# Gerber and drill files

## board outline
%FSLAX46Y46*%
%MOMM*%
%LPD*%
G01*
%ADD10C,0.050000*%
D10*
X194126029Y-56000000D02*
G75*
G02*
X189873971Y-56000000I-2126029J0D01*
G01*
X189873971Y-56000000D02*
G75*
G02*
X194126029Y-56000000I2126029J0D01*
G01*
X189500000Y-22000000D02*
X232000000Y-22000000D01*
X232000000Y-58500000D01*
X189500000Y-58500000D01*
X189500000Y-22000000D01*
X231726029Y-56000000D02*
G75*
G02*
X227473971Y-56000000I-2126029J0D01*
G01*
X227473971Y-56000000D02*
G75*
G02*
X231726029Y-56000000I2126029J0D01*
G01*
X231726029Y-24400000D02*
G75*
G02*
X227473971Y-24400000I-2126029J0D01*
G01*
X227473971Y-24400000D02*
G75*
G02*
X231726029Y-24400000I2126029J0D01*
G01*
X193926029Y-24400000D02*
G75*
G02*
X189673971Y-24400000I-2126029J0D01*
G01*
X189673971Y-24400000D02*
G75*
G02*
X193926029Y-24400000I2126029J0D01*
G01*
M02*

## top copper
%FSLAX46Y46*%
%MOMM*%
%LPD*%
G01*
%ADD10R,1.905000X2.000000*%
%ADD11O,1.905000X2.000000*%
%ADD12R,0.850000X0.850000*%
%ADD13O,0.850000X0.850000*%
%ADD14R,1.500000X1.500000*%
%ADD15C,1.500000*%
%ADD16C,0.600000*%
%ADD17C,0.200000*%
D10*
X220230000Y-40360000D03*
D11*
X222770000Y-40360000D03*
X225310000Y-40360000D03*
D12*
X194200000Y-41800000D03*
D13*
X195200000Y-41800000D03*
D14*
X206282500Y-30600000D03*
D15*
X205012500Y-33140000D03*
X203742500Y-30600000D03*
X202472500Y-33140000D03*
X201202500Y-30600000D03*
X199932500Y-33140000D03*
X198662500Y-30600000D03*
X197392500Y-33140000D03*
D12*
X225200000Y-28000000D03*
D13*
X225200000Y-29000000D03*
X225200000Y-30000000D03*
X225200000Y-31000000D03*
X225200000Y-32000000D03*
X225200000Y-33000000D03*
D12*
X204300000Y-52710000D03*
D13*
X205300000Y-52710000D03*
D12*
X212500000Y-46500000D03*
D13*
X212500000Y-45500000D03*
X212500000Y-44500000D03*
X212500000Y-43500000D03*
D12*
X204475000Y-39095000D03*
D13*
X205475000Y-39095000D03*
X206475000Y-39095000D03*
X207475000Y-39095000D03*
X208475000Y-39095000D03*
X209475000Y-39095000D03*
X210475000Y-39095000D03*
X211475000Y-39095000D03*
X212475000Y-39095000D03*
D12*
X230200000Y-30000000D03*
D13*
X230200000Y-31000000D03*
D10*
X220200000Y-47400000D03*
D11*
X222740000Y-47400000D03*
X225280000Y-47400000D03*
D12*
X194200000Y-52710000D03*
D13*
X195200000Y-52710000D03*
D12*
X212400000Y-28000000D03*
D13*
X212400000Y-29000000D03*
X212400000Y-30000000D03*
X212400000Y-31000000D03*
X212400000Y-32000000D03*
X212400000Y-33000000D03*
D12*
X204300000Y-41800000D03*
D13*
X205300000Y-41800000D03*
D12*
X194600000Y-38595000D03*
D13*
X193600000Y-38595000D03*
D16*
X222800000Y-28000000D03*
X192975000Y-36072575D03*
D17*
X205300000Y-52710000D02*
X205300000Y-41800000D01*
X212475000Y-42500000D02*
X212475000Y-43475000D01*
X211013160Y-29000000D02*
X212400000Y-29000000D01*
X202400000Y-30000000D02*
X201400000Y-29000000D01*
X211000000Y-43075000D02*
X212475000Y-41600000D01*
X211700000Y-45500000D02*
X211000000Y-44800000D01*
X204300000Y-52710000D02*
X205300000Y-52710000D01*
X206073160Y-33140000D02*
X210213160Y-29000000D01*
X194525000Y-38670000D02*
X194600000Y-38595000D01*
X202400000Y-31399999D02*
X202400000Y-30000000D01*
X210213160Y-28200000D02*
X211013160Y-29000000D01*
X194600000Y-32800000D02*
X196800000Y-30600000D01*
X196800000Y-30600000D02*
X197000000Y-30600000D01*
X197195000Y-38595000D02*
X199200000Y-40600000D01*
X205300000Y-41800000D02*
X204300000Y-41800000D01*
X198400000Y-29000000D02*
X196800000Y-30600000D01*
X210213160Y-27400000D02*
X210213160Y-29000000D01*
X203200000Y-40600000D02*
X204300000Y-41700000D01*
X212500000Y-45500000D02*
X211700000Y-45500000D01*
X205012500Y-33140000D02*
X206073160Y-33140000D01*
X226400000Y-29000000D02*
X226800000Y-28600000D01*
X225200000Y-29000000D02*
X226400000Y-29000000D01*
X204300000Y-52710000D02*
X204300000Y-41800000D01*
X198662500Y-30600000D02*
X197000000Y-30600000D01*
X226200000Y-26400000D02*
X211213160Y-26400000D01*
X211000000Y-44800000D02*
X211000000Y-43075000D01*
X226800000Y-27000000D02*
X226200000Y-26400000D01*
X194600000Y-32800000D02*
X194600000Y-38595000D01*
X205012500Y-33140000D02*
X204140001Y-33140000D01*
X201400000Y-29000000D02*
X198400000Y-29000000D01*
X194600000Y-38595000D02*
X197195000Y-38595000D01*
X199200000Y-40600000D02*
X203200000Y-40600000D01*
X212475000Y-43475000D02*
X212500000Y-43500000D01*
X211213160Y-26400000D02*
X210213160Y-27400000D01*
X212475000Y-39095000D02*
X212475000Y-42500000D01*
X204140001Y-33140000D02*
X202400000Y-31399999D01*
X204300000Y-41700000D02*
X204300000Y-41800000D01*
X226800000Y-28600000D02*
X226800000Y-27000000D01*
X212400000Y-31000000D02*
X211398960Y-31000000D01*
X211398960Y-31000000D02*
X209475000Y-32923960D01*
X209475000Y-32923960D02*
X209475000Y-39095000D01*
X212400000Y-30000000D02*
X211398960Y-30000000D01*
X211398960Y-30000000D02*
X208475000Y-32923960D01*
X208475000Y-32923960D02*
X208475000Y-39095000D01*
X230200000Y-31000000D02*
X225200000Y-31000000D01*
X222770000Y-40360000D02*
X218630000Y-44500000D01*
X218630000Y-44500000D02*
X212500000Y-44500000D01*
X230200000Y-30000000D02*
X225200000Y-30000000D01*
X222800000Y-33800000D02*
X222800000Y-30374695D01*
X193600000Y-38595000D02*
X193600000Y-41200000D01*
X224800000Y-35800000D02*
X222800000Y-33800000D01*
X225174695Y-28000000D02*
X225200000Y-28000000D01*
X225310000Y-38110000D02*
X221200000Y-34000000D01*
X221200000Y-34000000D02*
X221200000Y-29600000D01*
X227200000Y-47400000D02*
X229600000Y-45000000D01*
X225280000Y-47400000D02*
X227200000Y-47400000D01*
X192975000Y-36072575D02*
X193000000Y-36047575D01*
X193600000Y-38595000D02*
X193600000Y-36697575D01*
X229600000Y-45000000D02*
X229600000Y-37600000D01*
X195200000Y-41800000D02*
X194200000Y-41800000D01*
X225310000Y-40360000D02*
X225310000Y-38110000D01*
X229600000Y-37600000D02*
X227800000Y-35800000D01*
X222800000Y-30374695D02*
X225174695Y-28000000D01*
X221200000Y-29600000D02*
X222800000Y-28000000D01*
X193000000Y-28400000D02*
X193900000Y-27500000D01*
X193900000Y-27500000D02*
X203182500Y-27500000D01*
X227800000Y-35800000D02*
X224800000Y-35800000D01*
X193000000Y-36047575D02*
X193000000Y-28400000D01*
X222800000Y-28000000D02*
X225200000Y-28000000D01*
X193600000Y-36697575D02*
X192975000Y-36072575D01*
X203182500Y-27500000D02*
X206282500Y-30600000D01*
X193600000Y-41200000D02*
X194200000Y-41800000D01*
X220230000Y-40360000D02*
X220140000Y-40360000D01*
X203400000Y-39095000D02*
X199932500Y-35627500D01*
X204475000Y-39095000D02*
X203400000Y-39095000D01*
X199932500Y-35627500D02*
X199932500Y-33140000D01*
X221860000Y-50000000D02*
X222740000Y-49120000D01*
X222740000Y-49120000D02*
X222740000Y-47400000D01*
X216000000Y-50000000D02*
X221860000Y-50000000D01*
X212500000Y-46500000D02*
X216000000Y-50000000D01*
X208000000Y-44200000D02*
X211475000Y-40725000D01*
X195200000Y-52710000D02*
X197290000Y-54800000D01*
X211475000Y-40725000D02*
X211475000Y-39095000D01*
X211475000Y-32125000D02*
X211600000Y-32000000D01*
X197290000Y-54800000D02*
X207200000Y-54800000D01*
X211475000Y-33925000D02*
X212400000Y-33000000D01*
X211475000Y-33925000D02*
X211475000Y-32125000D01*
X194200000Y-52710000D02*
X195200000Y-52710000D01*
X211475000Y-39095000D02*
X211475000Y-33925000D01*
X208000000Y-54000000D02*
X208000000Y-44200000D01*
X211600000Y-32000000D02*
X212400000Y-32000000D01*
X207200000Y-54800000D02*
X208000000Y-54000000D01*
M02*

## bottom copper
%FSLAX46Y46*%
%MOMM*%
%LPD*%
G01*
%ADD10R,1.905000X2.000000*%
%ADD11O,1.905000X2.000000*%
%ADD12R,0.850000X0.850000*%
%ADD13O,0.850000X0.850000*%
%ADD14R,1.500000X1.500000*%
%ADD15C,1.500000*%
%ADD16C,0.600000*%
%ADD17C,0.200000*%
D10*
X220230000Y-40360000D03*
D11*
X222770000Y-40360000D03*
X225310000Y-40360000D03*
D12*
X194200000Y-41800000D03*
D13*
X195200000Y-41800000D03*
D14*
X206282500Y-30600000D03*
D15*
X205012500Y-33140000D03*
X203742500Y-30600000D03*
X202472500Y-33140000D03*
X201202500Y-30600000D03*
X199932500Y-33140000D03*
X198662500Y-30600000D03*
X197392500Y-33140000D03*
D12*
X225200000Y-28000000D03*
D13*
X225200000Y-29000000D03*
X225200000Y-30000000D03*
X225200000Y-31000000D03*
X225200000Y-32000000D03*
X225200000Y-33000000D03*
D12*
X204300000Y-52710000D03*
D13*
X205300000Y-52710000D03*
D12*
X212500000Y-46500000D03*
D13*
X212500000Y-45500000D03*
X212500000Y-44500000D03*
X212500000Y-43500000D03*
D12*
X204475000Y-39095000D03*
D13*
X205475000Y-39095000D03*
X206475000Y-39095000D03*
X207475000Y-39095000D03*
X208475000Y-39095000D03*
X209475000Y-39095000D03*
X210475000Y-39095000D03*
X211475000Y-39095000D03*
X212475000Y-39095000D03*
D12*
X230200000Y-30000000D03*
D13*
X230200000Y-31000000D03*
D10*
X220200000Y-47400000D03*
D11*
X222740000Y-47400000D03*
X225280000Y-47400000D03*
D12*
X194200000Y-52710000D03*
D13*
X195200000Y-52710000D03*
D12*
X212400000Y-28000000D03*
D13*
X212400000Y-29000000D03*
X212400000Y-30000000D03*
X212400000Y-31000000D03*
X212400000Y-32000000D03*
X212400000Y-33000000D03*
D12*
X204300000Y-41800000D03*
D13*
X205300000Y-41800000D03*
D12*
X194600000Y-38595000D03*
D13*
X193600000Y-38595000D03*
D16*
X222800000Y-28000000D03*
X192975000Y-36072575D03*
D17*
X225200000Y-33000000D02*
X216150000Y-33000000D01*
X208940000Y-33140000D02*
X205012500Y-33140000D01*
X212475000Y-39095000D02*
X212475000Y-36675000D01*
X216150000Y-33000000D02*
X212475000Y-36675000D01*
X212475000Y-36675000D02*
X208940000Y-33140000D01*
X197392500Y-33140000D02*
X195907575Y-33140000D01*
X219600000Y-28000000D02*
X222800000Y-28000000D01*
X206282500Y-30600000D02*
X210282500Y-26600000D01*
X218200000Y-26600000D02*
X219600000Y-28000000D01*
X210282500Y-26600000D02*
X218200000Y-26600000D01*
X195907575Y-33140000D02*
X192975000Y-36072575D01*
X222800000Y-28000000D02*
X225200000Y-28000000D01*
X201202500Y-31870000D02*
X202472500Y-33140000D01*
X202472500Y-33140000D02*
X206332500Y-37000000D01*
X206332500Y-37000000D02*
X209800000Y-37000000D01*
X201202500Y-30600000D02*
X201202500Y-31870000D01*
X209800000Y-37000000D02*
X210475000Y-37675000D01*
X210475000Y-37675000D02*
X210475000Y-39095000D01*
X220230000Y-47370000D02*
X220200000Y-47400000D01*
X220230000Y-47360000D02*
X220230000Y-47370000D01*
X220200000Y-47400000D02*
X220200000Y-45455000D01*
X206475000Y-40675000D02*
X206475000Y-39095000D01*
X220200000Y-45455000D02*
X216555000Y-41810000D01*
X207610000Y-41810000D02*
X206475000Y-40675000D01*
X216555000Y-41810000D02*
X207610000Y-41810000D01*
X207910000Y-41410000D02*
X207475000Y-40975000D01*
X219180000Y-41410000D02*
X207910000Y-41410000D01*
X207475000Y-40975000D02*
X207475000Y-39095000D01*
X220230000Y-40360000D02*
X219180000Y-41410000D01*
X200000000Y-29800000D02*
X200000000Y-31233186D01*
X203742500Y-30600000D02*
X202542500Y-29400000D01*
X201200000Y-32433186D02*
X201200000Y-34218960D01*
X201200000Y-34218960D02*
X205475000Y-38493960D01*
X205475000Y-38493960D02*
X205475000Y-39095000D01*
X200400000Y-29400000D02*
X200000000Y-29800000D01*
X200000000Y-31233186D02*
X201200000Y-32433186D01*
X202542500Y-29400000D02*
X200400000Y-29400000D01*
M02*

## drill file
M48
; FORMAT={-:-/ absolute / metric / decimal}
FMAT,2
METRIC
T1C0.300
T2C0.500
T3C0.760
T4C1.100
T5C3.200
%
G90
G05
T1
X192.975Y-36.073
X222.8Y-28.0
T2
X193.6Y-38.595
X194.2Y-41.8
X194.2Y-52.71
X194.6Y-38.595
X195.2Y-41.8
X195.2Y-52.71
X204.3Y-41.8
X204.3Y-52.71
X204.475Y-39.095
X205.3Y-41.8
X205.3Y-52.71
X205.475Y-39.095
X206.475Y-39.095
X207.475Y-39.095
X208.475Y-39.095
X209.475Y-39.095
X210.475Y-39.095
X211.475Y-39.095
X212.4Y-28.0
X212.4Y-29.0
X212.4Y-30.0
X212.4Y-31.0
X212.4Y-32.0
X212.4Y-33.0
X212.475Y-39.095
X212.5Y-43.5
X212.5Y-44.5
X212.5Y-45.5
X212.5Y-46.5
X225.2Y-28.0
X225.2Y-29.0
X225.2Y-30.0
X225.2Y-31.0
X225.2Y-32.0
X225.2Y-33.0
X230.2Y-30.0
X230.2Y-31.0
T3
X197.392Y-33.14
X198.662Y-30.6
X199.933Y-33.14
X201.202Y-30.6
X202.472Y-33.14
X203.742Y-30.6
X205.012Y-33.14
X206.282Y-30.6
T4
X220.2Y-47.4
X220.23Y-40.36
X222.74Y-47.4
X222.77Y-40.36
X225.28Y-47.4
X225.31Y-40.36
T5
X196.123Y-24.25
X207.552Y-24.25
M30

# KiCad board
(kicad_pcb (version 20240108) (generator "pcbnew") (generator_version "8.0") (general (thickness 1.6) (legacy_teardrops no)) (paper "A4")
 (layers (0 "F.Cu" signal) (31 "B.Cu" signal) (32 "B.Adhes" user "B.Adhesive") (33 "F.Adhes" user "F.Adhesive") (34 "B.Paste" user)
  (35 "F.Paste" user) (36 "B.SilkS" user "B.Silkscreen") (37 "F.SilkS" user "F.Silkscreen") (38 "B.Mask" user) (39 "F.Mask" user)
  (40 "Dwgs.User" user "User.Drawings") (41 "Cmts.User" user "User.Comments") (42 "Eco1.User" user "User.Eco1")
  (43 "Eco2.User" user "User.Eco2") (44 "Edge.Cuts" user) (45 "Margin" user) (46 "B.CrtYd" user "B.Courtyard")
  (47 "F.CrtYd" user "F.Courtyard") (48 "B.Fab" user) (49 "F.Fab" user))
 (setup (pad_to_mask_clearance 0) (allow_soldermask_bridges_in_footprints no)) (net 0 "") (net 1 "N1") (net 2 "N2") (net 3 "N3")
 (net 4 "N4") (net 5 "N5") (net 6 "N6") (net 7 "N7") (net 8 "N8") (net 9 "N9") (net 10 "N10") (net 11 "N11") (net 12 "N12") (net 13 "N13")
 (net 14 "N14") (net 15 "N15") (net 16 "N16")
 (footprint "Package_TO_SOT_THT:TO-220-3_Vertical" (layer "F.Cu") (at 220.23 40.36)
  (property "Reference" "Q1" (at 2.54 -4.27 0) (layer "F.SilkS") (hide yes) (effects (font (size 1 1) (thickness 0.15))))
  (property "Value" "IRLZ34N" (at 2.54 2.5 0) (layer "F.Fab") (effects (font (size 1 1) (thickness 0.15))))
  (pad "1" thru_hole rect (at 0 0) (size 1.905 2) (drill 1.1) (layers "*.Cu" "*.Mask") (remove_unused_layers no) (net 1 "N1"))
  (pad "2" thru_hole oval (at 2.54 0) (size 1.905 2) (drill 1.1) (layers "*.Cu" "*.Mask") (remove_unused_layers no) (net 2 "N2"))
  (pad "3" thru_hole oval (at 5.08 0) (size 1.905 2) (drill 1.1) (layers "*.Cu" "*.Mask") (remove_unused_layers no) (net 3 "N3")))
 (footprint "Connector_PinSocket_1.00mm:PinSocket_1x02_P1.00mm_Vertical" (layer "F.Cu") (at 194.2 41.8 90)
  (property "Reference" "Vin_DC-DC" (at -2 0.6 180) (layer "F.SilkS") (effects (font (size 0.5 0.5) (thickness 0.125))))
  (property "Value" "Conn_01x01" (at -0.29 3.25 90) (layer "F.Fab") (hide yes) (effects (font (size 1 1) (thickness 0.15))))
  (pad "1" thru_hole rect (at 0 0 90) (size 0.85 0.85) (drill 0.5) (layers "*.Cu" "*.Mask") (remove_unused_layers no) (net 3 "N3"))
  (pad "2" thru_hole oval (at 0 1 90) (size 0.85 0.85) (drill 0.5) (layers "*.Cu" "*.Mask") (remove_unused_layers no) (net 3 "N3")))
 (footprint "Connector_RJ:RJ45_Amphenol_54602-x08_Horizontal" (layer "F.Cu") (at 206.2825 30.6 180)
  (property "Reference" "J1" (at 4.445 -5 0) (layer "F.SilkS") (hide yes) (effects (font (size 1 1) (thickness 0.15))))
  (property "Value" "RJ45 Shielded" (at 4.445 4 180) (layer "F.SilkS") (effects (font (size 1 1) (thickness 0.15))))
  (pad "" np_thru_hole circle (at -1.27 6.35 180) (size 3.2 3.2) (drill 3.2) (layers "*.Cu" "*.Mask"))
  (pad "" np_thru_hole circle (at 10.16 6.35 180) (size 3.2 3.2) (drill 3.2) (layers "*.Cu" "*.Mask"))
  (pad "1" thru_hole rect (at 0 0 180) (size 1.5 1.5) (drill 0.76) (layers "*.Cu" "*.Mask") (remove_unused_layers no) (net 3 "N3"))
  (pad "2" thru_hole circle (at 1.27 -2.54 180) (size 1.5 1.5) (drill 0.76) (layers "*.Cu" "*.Mask") (remove_unused_layers no) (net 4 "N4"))
  (pad "3" thru_hole circle (at 2.54 0 180) (size 1.5 1.5) (drill 0.76) (layers "*.Cu" "*.Mask") (remove_unused_layers no) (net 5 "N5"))
  (pad "4" thru_hole circle (at 3.81 -2.54 180) (size 1.5 1.5) (drill 0.76) (layers "*.Cu" "*.Mask") (remove_unused_layers no) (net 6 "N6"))
  (pad "5" thru_hole circle (at 5.08 0 180) (size 1.5 1.5) (drill 0.76) (layers "*.Cu" "*.Mask") (remove_unused_layers no) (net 6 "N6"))
  (pad "6" thru_hole circle (at 6.35 -2.54 180) (size 1.5 1.5) (drill 0.76) (layers "*.Cu" "*.Mask") (remove_unused_layers no) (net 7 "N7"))
  (pad "7" thru_hole circle (at 7.62 0 180) (size 1.5 1.5) (drill 0.76) (layers "*.Cu" "*.Mask") (remove_unused_layers no) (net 4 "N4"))
  (pad "8" thru_hole circle (at 8.89 -2.54 180) (size 1.5 1.5) (drill 0.76) (layers "*.Cu" "*.Mask") (remove_unused_layers no) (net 3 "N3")))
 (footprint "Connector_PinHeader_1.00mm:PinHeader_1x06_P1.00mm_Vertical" (layer "F.Cu") (at 225.2 28)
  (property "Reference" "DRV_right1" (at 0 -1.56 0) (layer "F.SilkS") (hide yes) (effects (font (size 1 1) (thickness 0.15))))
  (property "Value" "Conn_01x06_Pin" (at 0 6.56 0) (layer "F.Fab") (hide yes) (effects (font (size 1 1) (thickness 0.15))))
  (pad "1" thru_hole rect (at 0 0) (size 0.85 0.85) (drill 0.5) (layers "*.Cu" "*.Mask") (remove_unused_layers no) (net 3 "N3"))
  (pad "2" thru_hole oval (at 0 1) (size 0.85 0.85) (drill 0.5) (layers "*.Cu" "*.Mask") (remove_unused_layers no) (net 4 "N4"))
  (pad "3" thru_hole oval (at 0 2) (size 0.85 0.85) (drill 0.5) (layers "*.Cu" "*.Mask") (remove_unused_layers no) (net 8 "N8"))
  (pad "4" thru_hole oval (at 0 3) (size 0.85 0.85) (drill 0.5) (layers "*.Cu" "*.Mask") (remove_unused_layers no) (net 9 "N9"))
  (pad "5" thru_hole oval (at 0 4) (size 0.85 0.85) (drill 0.5) (layers "*.Cu" "*.Mask") (remove_unused_layers no) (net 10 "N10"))
  (pad "6" thru_hole oval (at 0 5) (size 0.85 0.85) (drill 0.5) (layers "*.Cu" "*.Mask") (remove_unused_layers no) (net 4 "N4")))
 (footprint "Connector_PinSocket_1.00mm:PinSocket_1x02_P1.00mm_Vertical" (layer "F.Cu") (at 204.3 52.71 90)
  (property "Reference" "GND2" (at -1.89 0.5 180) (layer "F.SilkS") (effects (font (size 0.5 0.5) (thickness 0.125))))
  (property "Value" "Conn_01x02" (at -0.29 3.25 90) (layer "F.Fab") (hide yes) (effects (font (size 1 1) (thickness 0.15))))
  (pad "1" thru_hole rect (at 0 0 90) (size 0.85 0.85) (drill 0.5) (layers "*.Cu" "*.Mask") (remove_unused_layers no) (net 4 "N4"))
  (pad "2" thru_hole oval (at 0 1 90) (size 0.85 0.85) (drill 0.5) (layers "*.Cu" "*.Mask") (remove_unused_layers no) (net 4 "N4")))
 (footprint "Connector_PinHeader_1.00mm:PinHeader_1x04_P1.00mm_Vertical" (layer "F.Cu") (at 212.5 46.5 180)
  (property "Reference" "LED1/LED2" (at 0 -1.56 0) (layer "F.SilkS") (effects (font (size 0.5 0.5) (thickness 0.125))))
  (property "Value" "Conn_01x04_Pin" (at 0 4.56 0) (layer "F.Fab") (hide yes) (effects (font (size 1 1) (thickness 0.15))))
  (pad "1" thru_hole rect (at 0 0 180) (size 0.85 0.85) (drill 0.5) (layers "*.Cu" "*.Mask") (remove_unused_layers no) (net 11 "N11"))
  (pad "2" thru_hole oval (at 0 1 180) (size 0.85 0.85) (drill 0.5) (layers "*.Cu" "*.Mask") (remove_unused_layers no) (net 4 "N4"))
  (pad "3" thru_hole oval (at 0 2 180) (size 0.85 0.85) (drill 0.5) (layers "*.Cu" "*.Mask") (remove_unused_layers no) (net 2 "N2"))
  (pad "4" thru_hole oval (at 0 3 180) (size 0.85 0.85) (drill 0.5) (layers "*.Cu" "*.Mask") (remove_unused_layers no) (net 4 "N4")))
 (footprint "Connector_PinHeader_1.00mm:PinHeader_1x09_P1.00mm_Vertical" (layer "F.Cu") (at 204.475 39.095 90)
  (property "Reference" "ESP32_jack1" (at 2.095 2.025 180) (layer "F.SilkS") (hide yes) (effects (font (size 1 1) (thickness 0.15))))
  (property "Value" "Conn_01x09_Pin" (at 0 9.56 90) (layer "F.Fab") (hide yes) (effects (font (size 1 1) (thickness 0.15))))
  (pad "1" thru_hole rect (at 0 0 90) (size 0.85 0.85) (drill 0.5) (layers "*.Cu" "*.Mask") (remove_unused_layers no) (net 7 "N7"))
  (pad "2" thru_hole oval (at 0 1 90) (size 0.85 0.85) (drill 0.5) (layers "*.Cu" "*.Mask") (remove_unused_layers no) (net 5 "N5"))
  (pad "3" thru_hole oval (at 0 2 90) (size 0.85 0.85) (drill 0.5) (layers "*.Cu" "*.Mask") (remove_unused_layers no) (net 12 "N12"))
  (pad "4" thru_hole oval (at 0 3 90) (size 0.85 0.85) (drill 0.5) (layers "*.Cu" "*.Mask") (remove_unused_layers no) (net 1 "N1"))
  (pad "5" thru_hole oval (at 0 4 90) (size 0.85 0.85) (drill 0.5) (layers "*.Cu" "*.Mask") (remove_unused_layers no) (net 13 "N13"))
  (pad "6" thru_hole oval (at 0 5 90) (size 0.85 0.85) (drill 0.5) (layers "*.Cu" "*.Mask") (remove_unused_layers no) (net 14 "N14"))
  (pad "7" thru_hole oval (at 0 6 90) (size 0.85 0.85) (drill 0.5) (layers "*.Cu" "*.Mask") (remove_unused_layers no) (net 6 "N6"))
  (pad "8" thru_hole oval (at 0 7 90) (size 0.85 0.85) (drill 0.5) (layers "*.Cu" "*.Mask") (remove_unused_layers no) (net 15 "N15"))
  (pad "9" thru_hole oval (at 0 8 90) (size 0.85 0.85) (drill 0.5) (layers "*.Cu" "*.Mask") (remove_unused_layers no) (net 4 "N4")))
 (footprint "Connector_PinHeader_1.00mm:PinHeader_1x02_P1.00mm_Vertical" (layer "F.Cu") (at 230.2 30)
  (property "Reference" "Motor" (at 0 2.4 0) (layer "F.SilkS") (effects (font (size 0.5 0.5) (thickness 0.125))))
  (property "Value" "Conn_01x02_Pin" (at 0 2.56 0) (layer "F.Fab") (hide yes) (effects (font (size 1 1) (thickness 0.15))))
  (pad "1" thru_hole rect (at 0 0) (size 0.85 0.85) (drill 0.5) (layers "*.Cu" "*.Mask") (remove_unused_layers no) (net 8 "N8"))
  (pad "2" thru_hole oval (at 0 1) (size 0.85 0.85) (drill 0.5) (layers "*.Cu" "*.Mask") (remove_unused_layers no) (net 9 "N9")))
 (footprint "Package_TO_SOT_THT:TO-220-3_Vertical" (layer "F.Cu") (at 220.2 47.4)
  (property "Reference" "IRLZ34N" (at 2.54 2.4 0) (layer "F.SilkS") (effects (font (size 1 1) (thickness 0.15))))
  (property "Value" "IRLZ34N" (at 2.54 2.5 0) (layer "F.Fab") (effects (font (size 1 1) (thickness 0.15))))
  (pad "1" thru_hole rect (at 0 0) (size 1.905 2) (drill 1.1) (layers "*.Cu" "*.Mask") (remove_unused_layers no) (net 12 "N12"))
  (pad "2" thru_hole oval (at 2.54 0) (size 1.905 2) (drill 1.1) (layers "*.Cu" "*.Mask") (remove_unused_layers no) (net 11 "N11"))
  (pad "3" thru_hole oval (at 5.08 0) (size 1.905 2) (drill 1.1) (layers "*.Cu" "*.Mask") (remove_unused_layers no) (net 3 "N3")))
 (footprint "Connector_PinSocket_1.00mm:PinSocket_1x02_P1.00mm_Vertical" (layer "F.Cu") (at 194.2 52.71 90)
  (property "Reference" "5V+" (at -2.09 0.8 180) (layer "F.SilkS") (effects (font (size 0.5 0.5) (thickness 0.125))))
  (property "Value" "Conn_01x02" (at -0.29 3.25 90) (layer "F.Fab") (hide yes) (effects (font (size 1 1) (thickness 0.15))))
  (pad "1" thru_hole rect (at 0 0 90) (size 0.85 0.85) (drill 0.5) (layers "*.Cu" "*.Mask") (remove_unused_layers no) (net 15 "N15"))
  (pad "2" thru_hole oval (at 0 1 90) (size 0.85 0.85) (drill 0.5) (layers "*.Cu" "*.Mask") (remove_unused_layers no) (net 15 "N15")))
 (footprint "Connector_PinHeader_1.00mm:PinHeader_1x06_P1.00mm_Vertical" (layer "F.Cu") (at 212.4 28)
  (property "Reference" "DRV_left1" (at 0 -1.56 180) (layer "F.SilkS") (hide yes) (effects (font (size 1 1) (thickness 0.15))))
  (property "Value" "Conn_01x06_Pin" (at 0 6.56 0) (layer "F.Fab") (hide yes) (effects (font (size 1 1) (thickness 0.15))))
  (pad "1" thru_hole rect (at 0 0) (size 0.85 0.85) (drill 0.5) (layers "*.Cu" "*.Mask") (remove_unused_layers no) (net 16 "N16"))
  (pad "2" thru_hole oval (at 0 1) (size 0.85 0.85) (drill 0.5) (layers "*.Cu" "*.Mask") (remove_unused_layers no) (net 4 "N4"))
  (pad "3" thru_hole oval (at 0 2) (size 0.85 0.85) (drill 0.5) (layers "*.Cu" "*.Mask") (remove_unused_layers no) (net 13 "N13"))
  (pad "4" thru_hole oval (at 0 3) (size 0.85 0.85) (drill 0.5) (layers "*.Cu" "*.Mask") (remove_unused_layers no) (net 14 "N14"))
  (pad "5" thru_hole oval (at 0 4) (size 0.85 0.85) (drill 0.5) (layers "*.Cu" "*.Mask") (remove_unused_layers no) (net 15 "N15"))
  (pad "6" thru_hole oval (at 0 5) (size 0.85 0.85) (drill 0.5) (layers "*.Cu" "*.Mask") (remove_unused_layers no) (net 15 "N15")))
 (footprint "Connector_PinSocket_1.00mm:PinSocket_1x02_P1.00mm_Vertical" (layer "F.Cu") (at 204.3 41.8 90)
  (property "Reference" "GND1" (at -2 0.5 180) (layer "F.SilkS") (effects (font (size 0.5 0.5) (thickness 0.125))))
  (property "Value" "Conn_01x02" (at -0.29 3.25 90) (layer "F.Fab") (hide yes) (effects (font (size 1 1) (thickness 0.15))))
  (pad "1" thru_hole rect (at 0 0 90) (size 0.85 0.85) (drill 0.5) (layers "*.Cu" "*.Mask") (remove_unused_layers no) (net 4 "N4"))
  (pad "2" thru_hole oval (at 0 1 90) (size 0.85 0.85) (drill 0.5) (layers "*.Cu" "*.Mask") (remove_unused_layers no) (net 4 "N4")))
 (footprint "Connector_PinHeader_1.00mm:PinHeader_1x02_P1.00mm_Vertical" (layer "F.Cu") (at 194.6 38.595 -90)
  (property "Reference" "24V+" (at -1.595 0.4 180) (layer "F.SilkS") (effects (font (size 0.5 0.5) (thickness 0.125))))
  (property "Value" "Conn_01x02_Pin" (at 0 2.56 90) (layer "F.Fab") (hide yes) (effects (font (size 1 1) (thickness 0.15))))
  (pad "1" thru_hole rect (at 0 0 270) (size 0.85 0.85) (drill 0.5) (layers "*.Cu" "*.Mask") (remove_unused_layers no) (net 4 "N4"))
  (pad "2" thru_hole oval (at 0 1 270) (size 0.85 0.85) (drill 0.5) (layers "*.Cu" "*.Mask") (remove_unused_layers no) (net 3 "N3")))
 (gr_circle (center 192 56) (end 190.6 54.4) (stroke (width 0.05) (type default)) (fill none) (layer "Edge.Cuts"))
 (gr_rect (start 189.5 22) (end 232 58.5) (stroke (width 0.05) (type default)) (fill none) (layer "Edge.Cuts"))
 (gr_circle (center 229.6 56) (end 228.2 54.4) (stroke (width 0.05) (type default)) (fill none) (layer "Edge.Cuts"))
 (gr_circle (center 229.6 24.4) (end 228.2 22.8) (stroke (width 0.05) (type default)) (fill none) (layer "Edge.Cuts"))
 (gr_circle (center 191.8 24.4) (end 190.4 22.8) (stroke (width 0.05) (type default)) (fill none) (layer "Edge.Cuts"))
 (segment (start 205.3 52.71) (end 205.3 41.8) (width 0.2) (layer "F.Cu") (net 4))
 (segment (start 212.475 42.5) (end 212.475 43.475) (width 0.2) (layer "F.Cu") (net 4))
 (segment (start 211.01316 29) (end 212.4 29) (width 0.2) (layer "F.Cu") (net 4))
 (segment (start 202.4 30) (end 201.4 29) (width 0.2) (layer "F.Cu") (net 4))
 (segment (start 211 43.075) (end 212.475 41.6) (width 0.2) (layer "F.Cu") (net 4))
 (segment (start 211.7 45.5) (end 211 44.8) (width 0.2) (layer "F.Cu") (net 4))
 (segment (start 204.3 52.71) (end 205.3 52.71) (width 0.2) (layer "F.Cu") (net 4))
 (segment (start 206.07316 33.14) (end 210.21316 29) (width 0.2) (layer "F.Cu") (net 4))
 (segment (start 194.525 38.67) (end 194.6 38.595) (width 0.2) (layer "F.Cu") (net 4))
 (segment (start 202.4 31.399999) (end 202.4 30) (width 0.2) (layer "F.Cu") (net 4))
 (segment (start 210.21316 28.2) (end 211.01316 29) (width 0.2) (layer "F.Cu") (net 4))
 (segment (start 194.6 32.8) (end 196.8 30.6) (width 0.2) (layer "F.Cu") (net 4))
 (segment (start 196.8 30.6) (end 197 30.6) (width 0.2) (layer "F.Cu") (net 4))
 (segment (start 197.195 38.595) (end 199.2 40.6) (width 0.2) (layer "F.Cu") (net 4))
 (segment (start 205.3 41.8) (end 204.3 41.8) (width 0.2) (layer "F.Cu") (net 4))
 (segment (start 198.4 29) (end 196.8 30.6) (width 0.2) (layer "F.Cu") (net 4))
 (segment (start 210.21316 27.4) (end 210.21316 29) (width 0.2) (layer "F.Cu") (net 4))
 (segment (start 203.2 40.6) (end 204.3 41.7) (width 0.2) (layer "F.Cu") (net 4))
 (segment (start 212.5 45.5) (end 211.7 45.5) (width 0.2) (layer "F.Cu") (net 4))
 (segment (start 205.0125 33.14) (end 206.07316 33.14) (width 0.2) (layer "F.Cu") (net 4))
 (segment (start 226.4 29) (end 226.8 28.6) (width 0.2) (layer "F.Cu") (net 4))
 (segment (start 225.2 29) (end 226.4 29) (width 0.2) (layer "F.Cu") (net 4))
 (segment (start 204.3 52.71) (end 204.3 41.8) (width 0.2) (layer "F.Cu") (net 4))
 (segment (start 198.6625 30.6) (end 197 30.6) (width 0.2) (layer "F.Cu") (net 4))
 (segment (start 226.2 26.4) (end 211.21316 26.4) (width 0.2) (layer "F.Cu") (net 4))
 (segment (start 211 44.8) (end 211 43.075) (width 0.2) (layer "F.Cu") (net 4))
 (segment (start 226.8 27) (end 226.2 26.4) (width 0.2) (layer "F.Cu") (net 4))
 (segment (start 194.6 32.8) (end 194.6 38.595) (width 0.2) (layer "F.Cu") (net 4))
 (segment (start 205.0125 33.14) (end 204.140001 33.14) (width 0.2) (layer "F.Cu") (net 4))
 (segment (start 201.4 29) (end 198.4 29) (width 0.2) (layer "F.Cu") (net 4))
 (segment (start 194.6 38.595) (end 197.195 38.595) (width 0.2) (layer "F.Cu") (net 4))
 (segment (start 199.2 40.6) (end 203.2 40.6) (width 0.2) (layer "F.Cu") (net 4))
 (segment (start 212.475 43.475) (end 212.5 43.5) (width 0.2) (layer "F.Cu") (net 4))
 (segment (start 211.21316 26.4) (end 210.21316 27.4) (width 0.2) (layer "F.Cu") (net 4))
 (segment (start 212.475 39.095) (end 212.475 42.5) (width 0.2) (layer "F.Cu") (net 4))
 (segment (start 204.140001 33.14) (end 202.4 31.399999) (width 0.2) (layer "F.Cu") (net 4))
 (segment (start 204.3 41.7) (end 204.3 41.8) (width 0.2) (layer "F.Cu") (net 4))
 (segment (start 226.8 28.6) (end 226.8 27) (width 0.2) (layer "F.Cu") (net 4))
 (segment (start 225.2 33) (end 216.15 33) (width 0.2) (layer "B.Cu") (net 4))
 (segment (start 208.94 33.14) (end 205.0125 33.14) (width 0.2) (layer "B.Cu") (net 4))
 (segment (start 212.475 39.095) (end 212.475 36.675) (width 0.2) (layer "B.Cu") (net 4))
 (segment (start 216.15 33) (end 212.475 36.675) (width 0.2) (layer "B.Cu") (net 4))
 (segment (start 212.475 36.675) (end 208.94 33.14) (width 0.2) (layer "B.Cu") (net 4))
 (segment (start 212.4 31) (end 211.39896 31) (width 0.2) (layer "F.Cu") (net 14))
 (segment (start 211.39896 31) (end 209.475 32.92396) (width 0.2) (layer "F.Cu") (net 14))
 (segment (start 209.475 32.92396) (end 209.475 39.095) (width 0.2) (layer "F.Cu") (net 14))
 (segment (start 212.4 30) (end 211.39896 30) (width 0.2) (layer "F.Cu") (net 13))
 (segment (start 211.39896 30) (end 208.475 32.92396) (width 0.2) (layer "F.Cu") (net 13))
 (segment (start 208.475 32.92396) (end 208.475 39.095) (width 0.2) (layer "F.Cu") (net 13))
 (segment (start 230.2 31) (end 225.2 31) (width 0.2) (layer "F.Cu") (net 9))
 (segment (start 222.77 40.36) (end 218.63 44.5) (width 0.2) (layer "F.Cu") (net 2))
 (segment (start 218.63 44.5) (end 212.5 44.5) (width 0.2) (layer "F.Cu") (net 2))
 (segment (start 230.2 30) (end 225.2 30) (width 0.2) (layer "F.Cu") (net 8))
 (segment (start 222.8 33.8) (end 222.8 30.374695) (width 0.2) (layer "F.Cu") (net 3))
 (segment (start 193.6 38.595) (end 193.6 41.2) (width 0.2) (layer "F.Cu") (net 3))
 (segment (start 224.8 35.8) (end 222.8 33.8) (width 0.2) (layer "F.Cu") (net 3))
 (segment (start 225.174695 28) (end 225.2 28) (width 0.2) (layer "F.Cu") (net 3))
 (segment (start 225.31 38.11) (end 221.2 34) (width 0.2) (layer "F.Cu") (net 3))
 (segment (start 221.2 34) (end 221.2 29.6) (width 0.2) (layer "F.Cu") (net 3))
 (segment (start 227.2 47.4) (end 229.6 45) (width 0.2) (layer "F.Cu") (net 3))
 (segment (start 225.28 47.4) (end 227.2 47.4) (width 0.2) (layer "F.Cu") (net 3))
 (segment (start 192.975 36.072575) (end 193 36.047575) (width 0.2) (layer "F.Cu") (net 3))
 (segment (start 193.6 38.595) (end 193.6 36.697575) (width 0.2) (layer "F.Cu") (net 3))
 (segment (start 229.6 45) (end 229.6 37.6) (width 0.2) (layer "F.Cu") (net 3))
 (segment (start 195.2 41.8) (end 194.2 41.8) (width 0.2) (layer "F.Cu") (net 3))
 (segment (start 225.31 40.36) (end 225.31 38.11) (width 0.2) (layer "F.Cu") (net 3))
 (segment (start 229.6 37.6) (end 227.8 35.8) (width 0.2) (layer "F.Cu") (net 3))
 (segment (start 222.8 30.374695) (end 225.174695 28) (width 0.2) (layer "F.Cu") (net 3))
 (segment (start 221.2 29.6) (end 222.8 28) (width 0.2) (layer "F.Cu") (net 3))
 (segment (start 193 28.4) (end 193.9 27.5) (width 0.2) (layer "F.Cu") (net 3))
 (segment (start 193.9 27.5) (end 203.1825 27.5) (width 0.2) (layer "F.Cu") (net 3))
 (segment (start 227.8 35.8) (end 224.8 35.8) (width 0.2) (layer "F.Cu") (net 3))
 (segment (start 193 36.047575) (end 193 28.4) (width 0.2) (layer "F.Cu") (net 3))
 (segment (start 222.8 28) (end 225.2 28) (width 0.2) (layer "F.Cu") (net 3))
 (segment (start 193.6 36.697575) (end 192.975 36.072575) (width 0.2) (layer "F.Cu") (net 3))
 (segment (start 203.1825 27.5) (end 206.2825 30.6) (width 0.2) (layer "F.Cu") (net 3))
 (segment (start 193.6 41.2) (end 194.2 41.8) (width 0.2) (layer "F.Cu") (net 3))
 (via (at 222.8 28) (size 0.6) (drill 0.3) (layers "F.Cu" "B.Cu") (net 3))
 (via (at 192.975 36.072575) (size 0.6) (drill 0.3) (layers "F.Cu" "B.Cu") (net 3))
 (segment (start 197.3925 33.14) (end 195.907575 33.14) (width 0.2) (layer "B.Cu") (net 3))
 (segment (start 219.6 28) (end 222.8 28) (width 0.2) (layer "B.Cu") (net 3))
 (segment (start 206.2825 30.6) (end 210.2825 26.6) (width 0.2) (layer "B.Cu") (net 3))
 (segment (start 218.2 26.6) (end 219.6 28) (width 0.2) (layer "B.Cu") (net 3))
 (segment (start 210.2825 26.6) (end 218.2 26.6) (width 0.2) (layer "B.Cu") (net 3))
 (segment (start 195.907575 33.14) (end 192.975 36.072575) (width 0.2) (layer "B.Cu") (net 3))
 (segment (start 222.8 28) (end 225.2 28) (width 0.2) (layer "B.Cu") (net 3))
 (segment (start 201.2025 31.87) (end 202.4725 33.14) (width 0.2) (layer "B.Cu") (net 6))
 (segment (start 202.4725 33.14) (end 206.3325 37) (width 0.2) (layer "B.Cu") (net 6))
 (segment (start 206.3325 37) (end 209.8 37) (width 0.2) (layer "B.Cu") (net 6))
 (segment (start 201.2025 30.6) (end 201.2025 31.87) (width 0.2) (layer "B.Cu") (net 6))
 (segment (start 209.8 37) (end 210.475 37.675) (width 0.2) (layer "B.Cu") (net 6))
 (segment (start 210.475 37.675) (end 210.475 39.095) (width 0.2) (layer "B.Cu") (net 6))
 (segment (start 220.23 47.37) (end 220.2 47.4) (width 0.2) (layer "B.Cu") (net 12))
 (segment (start 220.23 47.36) (end 220.23 47.37) (width 0.2) (layer "B.Cu") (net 12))
 (segment (start 220.2 47.4) (end 220.2 45.455) (width 0.2) (layer "B.Cu") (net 12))
 (segment (start 206.475 40.675) (end 206.475 39.095) (width 0.2) (layer "B.Cu") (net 12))
 (segment (start 220.2 45.455) (end 216.555 41.81) (width 0.2) (layer "B.Cu") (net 12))
 (segment (start 207.61 41.81) (end 206.475 40.675) (width 0.2) (layer "B.Cu") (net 12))
 (segment (start 216.555 41.81) (end 207.61 41.81) (width 0.2) (layer "B.Cu") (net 12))
 (segment (start 220.23 40.36) (end 220.14 40.36) (width 0.2) (layer "F.Cu") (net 1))
 (segment (start 207.91 41.41) (end 207.475 40.975) (width 0.2) (layer "B.Cu") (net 1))
 (segment (start 219.18 41.41) (end 207.91 41.41) (width 0.2) (layer "B.Cu") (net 1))
 (segment (start 207.475 40.975) (end 207.475 39.095) (width 0.2) (layer "B.Cu") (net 1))
 (segment (start 220.23 40.36) (end 219.18 41.41) (width 0.2) (layer "B.Cu") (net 1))
 (segment (start 200 29.8) (end 200 31.233186) (width 0.2) (layer "B.Cu") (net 5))
 (segment (start 203.7425 30.6) (end 202.5425 29.4) (width 0.2) (layer "B.Cu") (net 5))
 (segment (start 201.2 32.433186) (end 201.2 34.21896) (width 0.2) (layer "B.Cu") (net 5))
 (segment (start 201.2 34.21896) (end 205.475 38.49396) (width 0.2) (layer "B.Cu") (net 5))
 (segment (start 205.475 38.49396) (end 205.475 39.095) (width 0.2) (layer "B.Cu") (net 5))
 (segment (start 200.4 29.4) (end 200 29.8) (width 0.2) (layer "B.Cu") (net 5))
 (segment (start 200 31.233186) (end 201.2 32.433186) (width 0.2) (layer "B.Cu") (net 5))
 (segment (start 202.5425 29.4) (end 200.4 29.4) (width 0.2) (layer "B.Cu") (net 5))
 (segment (start 203.4 39.095) (end 199.9325 35.6275) (width 0.2) (layer "F.Cu") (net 7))
 (segment (start 204.475 39.095) (end 203.4 39.095) (width 0.2) (layer "F.Cu") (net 7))
 (segment (start 199.9325 35.6275) (end 199.9325 33.14) (width 0.2) (layer "F.Cu") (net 7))
 (segment (start 221.86 50) (end 222.74 49.12) (width 0.2) (layer "F.Cu") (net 11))
 (segment (start 222.74 49.12) (end 222.74 47.4) (width 0.2) (layer "F.Cu") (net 11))
 (segment (start 216 50) (end 221.86 50) (width 0.2) (layer "F.Cu") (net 11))
 (segment (start 212.5 46.5) (end 216 50) (width 0.2) (layer "F.Cu") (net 11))
 (segment (start 208 44.2) (end 211.475 40.725) (width 0.2) (layer "F.Cu") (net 15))
 (segment (start 195.2 52.71) (end 197.29 54.8) (width 0.2) (layer "F.Cu") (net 15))
 (segment (start 211.475 40.725) (end 211.475 39.095) (width 0.2) (layer "F.Cu") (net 15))
 (segment (start 211.475 32.125) (end 211.6 32) (width 0.2) (layer "F.Cu") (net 15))
 (segment (start 197.29 54.8) (end 207.2 54.8) (width 0.2) (layer "F.Cu") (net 15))
 (segment (start 211.475 33.925) (end 212.4 33) (width 0.2) (layer "F.Cu") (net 15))
 (segment (start 211.475 33.925) (end 211.475 32.125) (width 0.2) (layer "F.Cu") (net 15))
 (segment (start 194.2 52.71) (end 195.2 52.71) (width 0.2) (layer "F.Cu") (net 15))
 (segment (start 211.475 39.095) (end 211.475 33.925) (width 0.2) (layer "F.Cu") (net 15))
 (segment (start 208 54) (end 208 44.2) (width 0.2) (layer "F.Cu") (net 15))
 (segment (start 211.6 32) (end 212.4 32) (width 0.2) (layer "F.Cu") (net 15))
 (segment (start 207.2 54.8) (end 208 54) (width 0.2) (layer "F.Cu") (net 15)))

